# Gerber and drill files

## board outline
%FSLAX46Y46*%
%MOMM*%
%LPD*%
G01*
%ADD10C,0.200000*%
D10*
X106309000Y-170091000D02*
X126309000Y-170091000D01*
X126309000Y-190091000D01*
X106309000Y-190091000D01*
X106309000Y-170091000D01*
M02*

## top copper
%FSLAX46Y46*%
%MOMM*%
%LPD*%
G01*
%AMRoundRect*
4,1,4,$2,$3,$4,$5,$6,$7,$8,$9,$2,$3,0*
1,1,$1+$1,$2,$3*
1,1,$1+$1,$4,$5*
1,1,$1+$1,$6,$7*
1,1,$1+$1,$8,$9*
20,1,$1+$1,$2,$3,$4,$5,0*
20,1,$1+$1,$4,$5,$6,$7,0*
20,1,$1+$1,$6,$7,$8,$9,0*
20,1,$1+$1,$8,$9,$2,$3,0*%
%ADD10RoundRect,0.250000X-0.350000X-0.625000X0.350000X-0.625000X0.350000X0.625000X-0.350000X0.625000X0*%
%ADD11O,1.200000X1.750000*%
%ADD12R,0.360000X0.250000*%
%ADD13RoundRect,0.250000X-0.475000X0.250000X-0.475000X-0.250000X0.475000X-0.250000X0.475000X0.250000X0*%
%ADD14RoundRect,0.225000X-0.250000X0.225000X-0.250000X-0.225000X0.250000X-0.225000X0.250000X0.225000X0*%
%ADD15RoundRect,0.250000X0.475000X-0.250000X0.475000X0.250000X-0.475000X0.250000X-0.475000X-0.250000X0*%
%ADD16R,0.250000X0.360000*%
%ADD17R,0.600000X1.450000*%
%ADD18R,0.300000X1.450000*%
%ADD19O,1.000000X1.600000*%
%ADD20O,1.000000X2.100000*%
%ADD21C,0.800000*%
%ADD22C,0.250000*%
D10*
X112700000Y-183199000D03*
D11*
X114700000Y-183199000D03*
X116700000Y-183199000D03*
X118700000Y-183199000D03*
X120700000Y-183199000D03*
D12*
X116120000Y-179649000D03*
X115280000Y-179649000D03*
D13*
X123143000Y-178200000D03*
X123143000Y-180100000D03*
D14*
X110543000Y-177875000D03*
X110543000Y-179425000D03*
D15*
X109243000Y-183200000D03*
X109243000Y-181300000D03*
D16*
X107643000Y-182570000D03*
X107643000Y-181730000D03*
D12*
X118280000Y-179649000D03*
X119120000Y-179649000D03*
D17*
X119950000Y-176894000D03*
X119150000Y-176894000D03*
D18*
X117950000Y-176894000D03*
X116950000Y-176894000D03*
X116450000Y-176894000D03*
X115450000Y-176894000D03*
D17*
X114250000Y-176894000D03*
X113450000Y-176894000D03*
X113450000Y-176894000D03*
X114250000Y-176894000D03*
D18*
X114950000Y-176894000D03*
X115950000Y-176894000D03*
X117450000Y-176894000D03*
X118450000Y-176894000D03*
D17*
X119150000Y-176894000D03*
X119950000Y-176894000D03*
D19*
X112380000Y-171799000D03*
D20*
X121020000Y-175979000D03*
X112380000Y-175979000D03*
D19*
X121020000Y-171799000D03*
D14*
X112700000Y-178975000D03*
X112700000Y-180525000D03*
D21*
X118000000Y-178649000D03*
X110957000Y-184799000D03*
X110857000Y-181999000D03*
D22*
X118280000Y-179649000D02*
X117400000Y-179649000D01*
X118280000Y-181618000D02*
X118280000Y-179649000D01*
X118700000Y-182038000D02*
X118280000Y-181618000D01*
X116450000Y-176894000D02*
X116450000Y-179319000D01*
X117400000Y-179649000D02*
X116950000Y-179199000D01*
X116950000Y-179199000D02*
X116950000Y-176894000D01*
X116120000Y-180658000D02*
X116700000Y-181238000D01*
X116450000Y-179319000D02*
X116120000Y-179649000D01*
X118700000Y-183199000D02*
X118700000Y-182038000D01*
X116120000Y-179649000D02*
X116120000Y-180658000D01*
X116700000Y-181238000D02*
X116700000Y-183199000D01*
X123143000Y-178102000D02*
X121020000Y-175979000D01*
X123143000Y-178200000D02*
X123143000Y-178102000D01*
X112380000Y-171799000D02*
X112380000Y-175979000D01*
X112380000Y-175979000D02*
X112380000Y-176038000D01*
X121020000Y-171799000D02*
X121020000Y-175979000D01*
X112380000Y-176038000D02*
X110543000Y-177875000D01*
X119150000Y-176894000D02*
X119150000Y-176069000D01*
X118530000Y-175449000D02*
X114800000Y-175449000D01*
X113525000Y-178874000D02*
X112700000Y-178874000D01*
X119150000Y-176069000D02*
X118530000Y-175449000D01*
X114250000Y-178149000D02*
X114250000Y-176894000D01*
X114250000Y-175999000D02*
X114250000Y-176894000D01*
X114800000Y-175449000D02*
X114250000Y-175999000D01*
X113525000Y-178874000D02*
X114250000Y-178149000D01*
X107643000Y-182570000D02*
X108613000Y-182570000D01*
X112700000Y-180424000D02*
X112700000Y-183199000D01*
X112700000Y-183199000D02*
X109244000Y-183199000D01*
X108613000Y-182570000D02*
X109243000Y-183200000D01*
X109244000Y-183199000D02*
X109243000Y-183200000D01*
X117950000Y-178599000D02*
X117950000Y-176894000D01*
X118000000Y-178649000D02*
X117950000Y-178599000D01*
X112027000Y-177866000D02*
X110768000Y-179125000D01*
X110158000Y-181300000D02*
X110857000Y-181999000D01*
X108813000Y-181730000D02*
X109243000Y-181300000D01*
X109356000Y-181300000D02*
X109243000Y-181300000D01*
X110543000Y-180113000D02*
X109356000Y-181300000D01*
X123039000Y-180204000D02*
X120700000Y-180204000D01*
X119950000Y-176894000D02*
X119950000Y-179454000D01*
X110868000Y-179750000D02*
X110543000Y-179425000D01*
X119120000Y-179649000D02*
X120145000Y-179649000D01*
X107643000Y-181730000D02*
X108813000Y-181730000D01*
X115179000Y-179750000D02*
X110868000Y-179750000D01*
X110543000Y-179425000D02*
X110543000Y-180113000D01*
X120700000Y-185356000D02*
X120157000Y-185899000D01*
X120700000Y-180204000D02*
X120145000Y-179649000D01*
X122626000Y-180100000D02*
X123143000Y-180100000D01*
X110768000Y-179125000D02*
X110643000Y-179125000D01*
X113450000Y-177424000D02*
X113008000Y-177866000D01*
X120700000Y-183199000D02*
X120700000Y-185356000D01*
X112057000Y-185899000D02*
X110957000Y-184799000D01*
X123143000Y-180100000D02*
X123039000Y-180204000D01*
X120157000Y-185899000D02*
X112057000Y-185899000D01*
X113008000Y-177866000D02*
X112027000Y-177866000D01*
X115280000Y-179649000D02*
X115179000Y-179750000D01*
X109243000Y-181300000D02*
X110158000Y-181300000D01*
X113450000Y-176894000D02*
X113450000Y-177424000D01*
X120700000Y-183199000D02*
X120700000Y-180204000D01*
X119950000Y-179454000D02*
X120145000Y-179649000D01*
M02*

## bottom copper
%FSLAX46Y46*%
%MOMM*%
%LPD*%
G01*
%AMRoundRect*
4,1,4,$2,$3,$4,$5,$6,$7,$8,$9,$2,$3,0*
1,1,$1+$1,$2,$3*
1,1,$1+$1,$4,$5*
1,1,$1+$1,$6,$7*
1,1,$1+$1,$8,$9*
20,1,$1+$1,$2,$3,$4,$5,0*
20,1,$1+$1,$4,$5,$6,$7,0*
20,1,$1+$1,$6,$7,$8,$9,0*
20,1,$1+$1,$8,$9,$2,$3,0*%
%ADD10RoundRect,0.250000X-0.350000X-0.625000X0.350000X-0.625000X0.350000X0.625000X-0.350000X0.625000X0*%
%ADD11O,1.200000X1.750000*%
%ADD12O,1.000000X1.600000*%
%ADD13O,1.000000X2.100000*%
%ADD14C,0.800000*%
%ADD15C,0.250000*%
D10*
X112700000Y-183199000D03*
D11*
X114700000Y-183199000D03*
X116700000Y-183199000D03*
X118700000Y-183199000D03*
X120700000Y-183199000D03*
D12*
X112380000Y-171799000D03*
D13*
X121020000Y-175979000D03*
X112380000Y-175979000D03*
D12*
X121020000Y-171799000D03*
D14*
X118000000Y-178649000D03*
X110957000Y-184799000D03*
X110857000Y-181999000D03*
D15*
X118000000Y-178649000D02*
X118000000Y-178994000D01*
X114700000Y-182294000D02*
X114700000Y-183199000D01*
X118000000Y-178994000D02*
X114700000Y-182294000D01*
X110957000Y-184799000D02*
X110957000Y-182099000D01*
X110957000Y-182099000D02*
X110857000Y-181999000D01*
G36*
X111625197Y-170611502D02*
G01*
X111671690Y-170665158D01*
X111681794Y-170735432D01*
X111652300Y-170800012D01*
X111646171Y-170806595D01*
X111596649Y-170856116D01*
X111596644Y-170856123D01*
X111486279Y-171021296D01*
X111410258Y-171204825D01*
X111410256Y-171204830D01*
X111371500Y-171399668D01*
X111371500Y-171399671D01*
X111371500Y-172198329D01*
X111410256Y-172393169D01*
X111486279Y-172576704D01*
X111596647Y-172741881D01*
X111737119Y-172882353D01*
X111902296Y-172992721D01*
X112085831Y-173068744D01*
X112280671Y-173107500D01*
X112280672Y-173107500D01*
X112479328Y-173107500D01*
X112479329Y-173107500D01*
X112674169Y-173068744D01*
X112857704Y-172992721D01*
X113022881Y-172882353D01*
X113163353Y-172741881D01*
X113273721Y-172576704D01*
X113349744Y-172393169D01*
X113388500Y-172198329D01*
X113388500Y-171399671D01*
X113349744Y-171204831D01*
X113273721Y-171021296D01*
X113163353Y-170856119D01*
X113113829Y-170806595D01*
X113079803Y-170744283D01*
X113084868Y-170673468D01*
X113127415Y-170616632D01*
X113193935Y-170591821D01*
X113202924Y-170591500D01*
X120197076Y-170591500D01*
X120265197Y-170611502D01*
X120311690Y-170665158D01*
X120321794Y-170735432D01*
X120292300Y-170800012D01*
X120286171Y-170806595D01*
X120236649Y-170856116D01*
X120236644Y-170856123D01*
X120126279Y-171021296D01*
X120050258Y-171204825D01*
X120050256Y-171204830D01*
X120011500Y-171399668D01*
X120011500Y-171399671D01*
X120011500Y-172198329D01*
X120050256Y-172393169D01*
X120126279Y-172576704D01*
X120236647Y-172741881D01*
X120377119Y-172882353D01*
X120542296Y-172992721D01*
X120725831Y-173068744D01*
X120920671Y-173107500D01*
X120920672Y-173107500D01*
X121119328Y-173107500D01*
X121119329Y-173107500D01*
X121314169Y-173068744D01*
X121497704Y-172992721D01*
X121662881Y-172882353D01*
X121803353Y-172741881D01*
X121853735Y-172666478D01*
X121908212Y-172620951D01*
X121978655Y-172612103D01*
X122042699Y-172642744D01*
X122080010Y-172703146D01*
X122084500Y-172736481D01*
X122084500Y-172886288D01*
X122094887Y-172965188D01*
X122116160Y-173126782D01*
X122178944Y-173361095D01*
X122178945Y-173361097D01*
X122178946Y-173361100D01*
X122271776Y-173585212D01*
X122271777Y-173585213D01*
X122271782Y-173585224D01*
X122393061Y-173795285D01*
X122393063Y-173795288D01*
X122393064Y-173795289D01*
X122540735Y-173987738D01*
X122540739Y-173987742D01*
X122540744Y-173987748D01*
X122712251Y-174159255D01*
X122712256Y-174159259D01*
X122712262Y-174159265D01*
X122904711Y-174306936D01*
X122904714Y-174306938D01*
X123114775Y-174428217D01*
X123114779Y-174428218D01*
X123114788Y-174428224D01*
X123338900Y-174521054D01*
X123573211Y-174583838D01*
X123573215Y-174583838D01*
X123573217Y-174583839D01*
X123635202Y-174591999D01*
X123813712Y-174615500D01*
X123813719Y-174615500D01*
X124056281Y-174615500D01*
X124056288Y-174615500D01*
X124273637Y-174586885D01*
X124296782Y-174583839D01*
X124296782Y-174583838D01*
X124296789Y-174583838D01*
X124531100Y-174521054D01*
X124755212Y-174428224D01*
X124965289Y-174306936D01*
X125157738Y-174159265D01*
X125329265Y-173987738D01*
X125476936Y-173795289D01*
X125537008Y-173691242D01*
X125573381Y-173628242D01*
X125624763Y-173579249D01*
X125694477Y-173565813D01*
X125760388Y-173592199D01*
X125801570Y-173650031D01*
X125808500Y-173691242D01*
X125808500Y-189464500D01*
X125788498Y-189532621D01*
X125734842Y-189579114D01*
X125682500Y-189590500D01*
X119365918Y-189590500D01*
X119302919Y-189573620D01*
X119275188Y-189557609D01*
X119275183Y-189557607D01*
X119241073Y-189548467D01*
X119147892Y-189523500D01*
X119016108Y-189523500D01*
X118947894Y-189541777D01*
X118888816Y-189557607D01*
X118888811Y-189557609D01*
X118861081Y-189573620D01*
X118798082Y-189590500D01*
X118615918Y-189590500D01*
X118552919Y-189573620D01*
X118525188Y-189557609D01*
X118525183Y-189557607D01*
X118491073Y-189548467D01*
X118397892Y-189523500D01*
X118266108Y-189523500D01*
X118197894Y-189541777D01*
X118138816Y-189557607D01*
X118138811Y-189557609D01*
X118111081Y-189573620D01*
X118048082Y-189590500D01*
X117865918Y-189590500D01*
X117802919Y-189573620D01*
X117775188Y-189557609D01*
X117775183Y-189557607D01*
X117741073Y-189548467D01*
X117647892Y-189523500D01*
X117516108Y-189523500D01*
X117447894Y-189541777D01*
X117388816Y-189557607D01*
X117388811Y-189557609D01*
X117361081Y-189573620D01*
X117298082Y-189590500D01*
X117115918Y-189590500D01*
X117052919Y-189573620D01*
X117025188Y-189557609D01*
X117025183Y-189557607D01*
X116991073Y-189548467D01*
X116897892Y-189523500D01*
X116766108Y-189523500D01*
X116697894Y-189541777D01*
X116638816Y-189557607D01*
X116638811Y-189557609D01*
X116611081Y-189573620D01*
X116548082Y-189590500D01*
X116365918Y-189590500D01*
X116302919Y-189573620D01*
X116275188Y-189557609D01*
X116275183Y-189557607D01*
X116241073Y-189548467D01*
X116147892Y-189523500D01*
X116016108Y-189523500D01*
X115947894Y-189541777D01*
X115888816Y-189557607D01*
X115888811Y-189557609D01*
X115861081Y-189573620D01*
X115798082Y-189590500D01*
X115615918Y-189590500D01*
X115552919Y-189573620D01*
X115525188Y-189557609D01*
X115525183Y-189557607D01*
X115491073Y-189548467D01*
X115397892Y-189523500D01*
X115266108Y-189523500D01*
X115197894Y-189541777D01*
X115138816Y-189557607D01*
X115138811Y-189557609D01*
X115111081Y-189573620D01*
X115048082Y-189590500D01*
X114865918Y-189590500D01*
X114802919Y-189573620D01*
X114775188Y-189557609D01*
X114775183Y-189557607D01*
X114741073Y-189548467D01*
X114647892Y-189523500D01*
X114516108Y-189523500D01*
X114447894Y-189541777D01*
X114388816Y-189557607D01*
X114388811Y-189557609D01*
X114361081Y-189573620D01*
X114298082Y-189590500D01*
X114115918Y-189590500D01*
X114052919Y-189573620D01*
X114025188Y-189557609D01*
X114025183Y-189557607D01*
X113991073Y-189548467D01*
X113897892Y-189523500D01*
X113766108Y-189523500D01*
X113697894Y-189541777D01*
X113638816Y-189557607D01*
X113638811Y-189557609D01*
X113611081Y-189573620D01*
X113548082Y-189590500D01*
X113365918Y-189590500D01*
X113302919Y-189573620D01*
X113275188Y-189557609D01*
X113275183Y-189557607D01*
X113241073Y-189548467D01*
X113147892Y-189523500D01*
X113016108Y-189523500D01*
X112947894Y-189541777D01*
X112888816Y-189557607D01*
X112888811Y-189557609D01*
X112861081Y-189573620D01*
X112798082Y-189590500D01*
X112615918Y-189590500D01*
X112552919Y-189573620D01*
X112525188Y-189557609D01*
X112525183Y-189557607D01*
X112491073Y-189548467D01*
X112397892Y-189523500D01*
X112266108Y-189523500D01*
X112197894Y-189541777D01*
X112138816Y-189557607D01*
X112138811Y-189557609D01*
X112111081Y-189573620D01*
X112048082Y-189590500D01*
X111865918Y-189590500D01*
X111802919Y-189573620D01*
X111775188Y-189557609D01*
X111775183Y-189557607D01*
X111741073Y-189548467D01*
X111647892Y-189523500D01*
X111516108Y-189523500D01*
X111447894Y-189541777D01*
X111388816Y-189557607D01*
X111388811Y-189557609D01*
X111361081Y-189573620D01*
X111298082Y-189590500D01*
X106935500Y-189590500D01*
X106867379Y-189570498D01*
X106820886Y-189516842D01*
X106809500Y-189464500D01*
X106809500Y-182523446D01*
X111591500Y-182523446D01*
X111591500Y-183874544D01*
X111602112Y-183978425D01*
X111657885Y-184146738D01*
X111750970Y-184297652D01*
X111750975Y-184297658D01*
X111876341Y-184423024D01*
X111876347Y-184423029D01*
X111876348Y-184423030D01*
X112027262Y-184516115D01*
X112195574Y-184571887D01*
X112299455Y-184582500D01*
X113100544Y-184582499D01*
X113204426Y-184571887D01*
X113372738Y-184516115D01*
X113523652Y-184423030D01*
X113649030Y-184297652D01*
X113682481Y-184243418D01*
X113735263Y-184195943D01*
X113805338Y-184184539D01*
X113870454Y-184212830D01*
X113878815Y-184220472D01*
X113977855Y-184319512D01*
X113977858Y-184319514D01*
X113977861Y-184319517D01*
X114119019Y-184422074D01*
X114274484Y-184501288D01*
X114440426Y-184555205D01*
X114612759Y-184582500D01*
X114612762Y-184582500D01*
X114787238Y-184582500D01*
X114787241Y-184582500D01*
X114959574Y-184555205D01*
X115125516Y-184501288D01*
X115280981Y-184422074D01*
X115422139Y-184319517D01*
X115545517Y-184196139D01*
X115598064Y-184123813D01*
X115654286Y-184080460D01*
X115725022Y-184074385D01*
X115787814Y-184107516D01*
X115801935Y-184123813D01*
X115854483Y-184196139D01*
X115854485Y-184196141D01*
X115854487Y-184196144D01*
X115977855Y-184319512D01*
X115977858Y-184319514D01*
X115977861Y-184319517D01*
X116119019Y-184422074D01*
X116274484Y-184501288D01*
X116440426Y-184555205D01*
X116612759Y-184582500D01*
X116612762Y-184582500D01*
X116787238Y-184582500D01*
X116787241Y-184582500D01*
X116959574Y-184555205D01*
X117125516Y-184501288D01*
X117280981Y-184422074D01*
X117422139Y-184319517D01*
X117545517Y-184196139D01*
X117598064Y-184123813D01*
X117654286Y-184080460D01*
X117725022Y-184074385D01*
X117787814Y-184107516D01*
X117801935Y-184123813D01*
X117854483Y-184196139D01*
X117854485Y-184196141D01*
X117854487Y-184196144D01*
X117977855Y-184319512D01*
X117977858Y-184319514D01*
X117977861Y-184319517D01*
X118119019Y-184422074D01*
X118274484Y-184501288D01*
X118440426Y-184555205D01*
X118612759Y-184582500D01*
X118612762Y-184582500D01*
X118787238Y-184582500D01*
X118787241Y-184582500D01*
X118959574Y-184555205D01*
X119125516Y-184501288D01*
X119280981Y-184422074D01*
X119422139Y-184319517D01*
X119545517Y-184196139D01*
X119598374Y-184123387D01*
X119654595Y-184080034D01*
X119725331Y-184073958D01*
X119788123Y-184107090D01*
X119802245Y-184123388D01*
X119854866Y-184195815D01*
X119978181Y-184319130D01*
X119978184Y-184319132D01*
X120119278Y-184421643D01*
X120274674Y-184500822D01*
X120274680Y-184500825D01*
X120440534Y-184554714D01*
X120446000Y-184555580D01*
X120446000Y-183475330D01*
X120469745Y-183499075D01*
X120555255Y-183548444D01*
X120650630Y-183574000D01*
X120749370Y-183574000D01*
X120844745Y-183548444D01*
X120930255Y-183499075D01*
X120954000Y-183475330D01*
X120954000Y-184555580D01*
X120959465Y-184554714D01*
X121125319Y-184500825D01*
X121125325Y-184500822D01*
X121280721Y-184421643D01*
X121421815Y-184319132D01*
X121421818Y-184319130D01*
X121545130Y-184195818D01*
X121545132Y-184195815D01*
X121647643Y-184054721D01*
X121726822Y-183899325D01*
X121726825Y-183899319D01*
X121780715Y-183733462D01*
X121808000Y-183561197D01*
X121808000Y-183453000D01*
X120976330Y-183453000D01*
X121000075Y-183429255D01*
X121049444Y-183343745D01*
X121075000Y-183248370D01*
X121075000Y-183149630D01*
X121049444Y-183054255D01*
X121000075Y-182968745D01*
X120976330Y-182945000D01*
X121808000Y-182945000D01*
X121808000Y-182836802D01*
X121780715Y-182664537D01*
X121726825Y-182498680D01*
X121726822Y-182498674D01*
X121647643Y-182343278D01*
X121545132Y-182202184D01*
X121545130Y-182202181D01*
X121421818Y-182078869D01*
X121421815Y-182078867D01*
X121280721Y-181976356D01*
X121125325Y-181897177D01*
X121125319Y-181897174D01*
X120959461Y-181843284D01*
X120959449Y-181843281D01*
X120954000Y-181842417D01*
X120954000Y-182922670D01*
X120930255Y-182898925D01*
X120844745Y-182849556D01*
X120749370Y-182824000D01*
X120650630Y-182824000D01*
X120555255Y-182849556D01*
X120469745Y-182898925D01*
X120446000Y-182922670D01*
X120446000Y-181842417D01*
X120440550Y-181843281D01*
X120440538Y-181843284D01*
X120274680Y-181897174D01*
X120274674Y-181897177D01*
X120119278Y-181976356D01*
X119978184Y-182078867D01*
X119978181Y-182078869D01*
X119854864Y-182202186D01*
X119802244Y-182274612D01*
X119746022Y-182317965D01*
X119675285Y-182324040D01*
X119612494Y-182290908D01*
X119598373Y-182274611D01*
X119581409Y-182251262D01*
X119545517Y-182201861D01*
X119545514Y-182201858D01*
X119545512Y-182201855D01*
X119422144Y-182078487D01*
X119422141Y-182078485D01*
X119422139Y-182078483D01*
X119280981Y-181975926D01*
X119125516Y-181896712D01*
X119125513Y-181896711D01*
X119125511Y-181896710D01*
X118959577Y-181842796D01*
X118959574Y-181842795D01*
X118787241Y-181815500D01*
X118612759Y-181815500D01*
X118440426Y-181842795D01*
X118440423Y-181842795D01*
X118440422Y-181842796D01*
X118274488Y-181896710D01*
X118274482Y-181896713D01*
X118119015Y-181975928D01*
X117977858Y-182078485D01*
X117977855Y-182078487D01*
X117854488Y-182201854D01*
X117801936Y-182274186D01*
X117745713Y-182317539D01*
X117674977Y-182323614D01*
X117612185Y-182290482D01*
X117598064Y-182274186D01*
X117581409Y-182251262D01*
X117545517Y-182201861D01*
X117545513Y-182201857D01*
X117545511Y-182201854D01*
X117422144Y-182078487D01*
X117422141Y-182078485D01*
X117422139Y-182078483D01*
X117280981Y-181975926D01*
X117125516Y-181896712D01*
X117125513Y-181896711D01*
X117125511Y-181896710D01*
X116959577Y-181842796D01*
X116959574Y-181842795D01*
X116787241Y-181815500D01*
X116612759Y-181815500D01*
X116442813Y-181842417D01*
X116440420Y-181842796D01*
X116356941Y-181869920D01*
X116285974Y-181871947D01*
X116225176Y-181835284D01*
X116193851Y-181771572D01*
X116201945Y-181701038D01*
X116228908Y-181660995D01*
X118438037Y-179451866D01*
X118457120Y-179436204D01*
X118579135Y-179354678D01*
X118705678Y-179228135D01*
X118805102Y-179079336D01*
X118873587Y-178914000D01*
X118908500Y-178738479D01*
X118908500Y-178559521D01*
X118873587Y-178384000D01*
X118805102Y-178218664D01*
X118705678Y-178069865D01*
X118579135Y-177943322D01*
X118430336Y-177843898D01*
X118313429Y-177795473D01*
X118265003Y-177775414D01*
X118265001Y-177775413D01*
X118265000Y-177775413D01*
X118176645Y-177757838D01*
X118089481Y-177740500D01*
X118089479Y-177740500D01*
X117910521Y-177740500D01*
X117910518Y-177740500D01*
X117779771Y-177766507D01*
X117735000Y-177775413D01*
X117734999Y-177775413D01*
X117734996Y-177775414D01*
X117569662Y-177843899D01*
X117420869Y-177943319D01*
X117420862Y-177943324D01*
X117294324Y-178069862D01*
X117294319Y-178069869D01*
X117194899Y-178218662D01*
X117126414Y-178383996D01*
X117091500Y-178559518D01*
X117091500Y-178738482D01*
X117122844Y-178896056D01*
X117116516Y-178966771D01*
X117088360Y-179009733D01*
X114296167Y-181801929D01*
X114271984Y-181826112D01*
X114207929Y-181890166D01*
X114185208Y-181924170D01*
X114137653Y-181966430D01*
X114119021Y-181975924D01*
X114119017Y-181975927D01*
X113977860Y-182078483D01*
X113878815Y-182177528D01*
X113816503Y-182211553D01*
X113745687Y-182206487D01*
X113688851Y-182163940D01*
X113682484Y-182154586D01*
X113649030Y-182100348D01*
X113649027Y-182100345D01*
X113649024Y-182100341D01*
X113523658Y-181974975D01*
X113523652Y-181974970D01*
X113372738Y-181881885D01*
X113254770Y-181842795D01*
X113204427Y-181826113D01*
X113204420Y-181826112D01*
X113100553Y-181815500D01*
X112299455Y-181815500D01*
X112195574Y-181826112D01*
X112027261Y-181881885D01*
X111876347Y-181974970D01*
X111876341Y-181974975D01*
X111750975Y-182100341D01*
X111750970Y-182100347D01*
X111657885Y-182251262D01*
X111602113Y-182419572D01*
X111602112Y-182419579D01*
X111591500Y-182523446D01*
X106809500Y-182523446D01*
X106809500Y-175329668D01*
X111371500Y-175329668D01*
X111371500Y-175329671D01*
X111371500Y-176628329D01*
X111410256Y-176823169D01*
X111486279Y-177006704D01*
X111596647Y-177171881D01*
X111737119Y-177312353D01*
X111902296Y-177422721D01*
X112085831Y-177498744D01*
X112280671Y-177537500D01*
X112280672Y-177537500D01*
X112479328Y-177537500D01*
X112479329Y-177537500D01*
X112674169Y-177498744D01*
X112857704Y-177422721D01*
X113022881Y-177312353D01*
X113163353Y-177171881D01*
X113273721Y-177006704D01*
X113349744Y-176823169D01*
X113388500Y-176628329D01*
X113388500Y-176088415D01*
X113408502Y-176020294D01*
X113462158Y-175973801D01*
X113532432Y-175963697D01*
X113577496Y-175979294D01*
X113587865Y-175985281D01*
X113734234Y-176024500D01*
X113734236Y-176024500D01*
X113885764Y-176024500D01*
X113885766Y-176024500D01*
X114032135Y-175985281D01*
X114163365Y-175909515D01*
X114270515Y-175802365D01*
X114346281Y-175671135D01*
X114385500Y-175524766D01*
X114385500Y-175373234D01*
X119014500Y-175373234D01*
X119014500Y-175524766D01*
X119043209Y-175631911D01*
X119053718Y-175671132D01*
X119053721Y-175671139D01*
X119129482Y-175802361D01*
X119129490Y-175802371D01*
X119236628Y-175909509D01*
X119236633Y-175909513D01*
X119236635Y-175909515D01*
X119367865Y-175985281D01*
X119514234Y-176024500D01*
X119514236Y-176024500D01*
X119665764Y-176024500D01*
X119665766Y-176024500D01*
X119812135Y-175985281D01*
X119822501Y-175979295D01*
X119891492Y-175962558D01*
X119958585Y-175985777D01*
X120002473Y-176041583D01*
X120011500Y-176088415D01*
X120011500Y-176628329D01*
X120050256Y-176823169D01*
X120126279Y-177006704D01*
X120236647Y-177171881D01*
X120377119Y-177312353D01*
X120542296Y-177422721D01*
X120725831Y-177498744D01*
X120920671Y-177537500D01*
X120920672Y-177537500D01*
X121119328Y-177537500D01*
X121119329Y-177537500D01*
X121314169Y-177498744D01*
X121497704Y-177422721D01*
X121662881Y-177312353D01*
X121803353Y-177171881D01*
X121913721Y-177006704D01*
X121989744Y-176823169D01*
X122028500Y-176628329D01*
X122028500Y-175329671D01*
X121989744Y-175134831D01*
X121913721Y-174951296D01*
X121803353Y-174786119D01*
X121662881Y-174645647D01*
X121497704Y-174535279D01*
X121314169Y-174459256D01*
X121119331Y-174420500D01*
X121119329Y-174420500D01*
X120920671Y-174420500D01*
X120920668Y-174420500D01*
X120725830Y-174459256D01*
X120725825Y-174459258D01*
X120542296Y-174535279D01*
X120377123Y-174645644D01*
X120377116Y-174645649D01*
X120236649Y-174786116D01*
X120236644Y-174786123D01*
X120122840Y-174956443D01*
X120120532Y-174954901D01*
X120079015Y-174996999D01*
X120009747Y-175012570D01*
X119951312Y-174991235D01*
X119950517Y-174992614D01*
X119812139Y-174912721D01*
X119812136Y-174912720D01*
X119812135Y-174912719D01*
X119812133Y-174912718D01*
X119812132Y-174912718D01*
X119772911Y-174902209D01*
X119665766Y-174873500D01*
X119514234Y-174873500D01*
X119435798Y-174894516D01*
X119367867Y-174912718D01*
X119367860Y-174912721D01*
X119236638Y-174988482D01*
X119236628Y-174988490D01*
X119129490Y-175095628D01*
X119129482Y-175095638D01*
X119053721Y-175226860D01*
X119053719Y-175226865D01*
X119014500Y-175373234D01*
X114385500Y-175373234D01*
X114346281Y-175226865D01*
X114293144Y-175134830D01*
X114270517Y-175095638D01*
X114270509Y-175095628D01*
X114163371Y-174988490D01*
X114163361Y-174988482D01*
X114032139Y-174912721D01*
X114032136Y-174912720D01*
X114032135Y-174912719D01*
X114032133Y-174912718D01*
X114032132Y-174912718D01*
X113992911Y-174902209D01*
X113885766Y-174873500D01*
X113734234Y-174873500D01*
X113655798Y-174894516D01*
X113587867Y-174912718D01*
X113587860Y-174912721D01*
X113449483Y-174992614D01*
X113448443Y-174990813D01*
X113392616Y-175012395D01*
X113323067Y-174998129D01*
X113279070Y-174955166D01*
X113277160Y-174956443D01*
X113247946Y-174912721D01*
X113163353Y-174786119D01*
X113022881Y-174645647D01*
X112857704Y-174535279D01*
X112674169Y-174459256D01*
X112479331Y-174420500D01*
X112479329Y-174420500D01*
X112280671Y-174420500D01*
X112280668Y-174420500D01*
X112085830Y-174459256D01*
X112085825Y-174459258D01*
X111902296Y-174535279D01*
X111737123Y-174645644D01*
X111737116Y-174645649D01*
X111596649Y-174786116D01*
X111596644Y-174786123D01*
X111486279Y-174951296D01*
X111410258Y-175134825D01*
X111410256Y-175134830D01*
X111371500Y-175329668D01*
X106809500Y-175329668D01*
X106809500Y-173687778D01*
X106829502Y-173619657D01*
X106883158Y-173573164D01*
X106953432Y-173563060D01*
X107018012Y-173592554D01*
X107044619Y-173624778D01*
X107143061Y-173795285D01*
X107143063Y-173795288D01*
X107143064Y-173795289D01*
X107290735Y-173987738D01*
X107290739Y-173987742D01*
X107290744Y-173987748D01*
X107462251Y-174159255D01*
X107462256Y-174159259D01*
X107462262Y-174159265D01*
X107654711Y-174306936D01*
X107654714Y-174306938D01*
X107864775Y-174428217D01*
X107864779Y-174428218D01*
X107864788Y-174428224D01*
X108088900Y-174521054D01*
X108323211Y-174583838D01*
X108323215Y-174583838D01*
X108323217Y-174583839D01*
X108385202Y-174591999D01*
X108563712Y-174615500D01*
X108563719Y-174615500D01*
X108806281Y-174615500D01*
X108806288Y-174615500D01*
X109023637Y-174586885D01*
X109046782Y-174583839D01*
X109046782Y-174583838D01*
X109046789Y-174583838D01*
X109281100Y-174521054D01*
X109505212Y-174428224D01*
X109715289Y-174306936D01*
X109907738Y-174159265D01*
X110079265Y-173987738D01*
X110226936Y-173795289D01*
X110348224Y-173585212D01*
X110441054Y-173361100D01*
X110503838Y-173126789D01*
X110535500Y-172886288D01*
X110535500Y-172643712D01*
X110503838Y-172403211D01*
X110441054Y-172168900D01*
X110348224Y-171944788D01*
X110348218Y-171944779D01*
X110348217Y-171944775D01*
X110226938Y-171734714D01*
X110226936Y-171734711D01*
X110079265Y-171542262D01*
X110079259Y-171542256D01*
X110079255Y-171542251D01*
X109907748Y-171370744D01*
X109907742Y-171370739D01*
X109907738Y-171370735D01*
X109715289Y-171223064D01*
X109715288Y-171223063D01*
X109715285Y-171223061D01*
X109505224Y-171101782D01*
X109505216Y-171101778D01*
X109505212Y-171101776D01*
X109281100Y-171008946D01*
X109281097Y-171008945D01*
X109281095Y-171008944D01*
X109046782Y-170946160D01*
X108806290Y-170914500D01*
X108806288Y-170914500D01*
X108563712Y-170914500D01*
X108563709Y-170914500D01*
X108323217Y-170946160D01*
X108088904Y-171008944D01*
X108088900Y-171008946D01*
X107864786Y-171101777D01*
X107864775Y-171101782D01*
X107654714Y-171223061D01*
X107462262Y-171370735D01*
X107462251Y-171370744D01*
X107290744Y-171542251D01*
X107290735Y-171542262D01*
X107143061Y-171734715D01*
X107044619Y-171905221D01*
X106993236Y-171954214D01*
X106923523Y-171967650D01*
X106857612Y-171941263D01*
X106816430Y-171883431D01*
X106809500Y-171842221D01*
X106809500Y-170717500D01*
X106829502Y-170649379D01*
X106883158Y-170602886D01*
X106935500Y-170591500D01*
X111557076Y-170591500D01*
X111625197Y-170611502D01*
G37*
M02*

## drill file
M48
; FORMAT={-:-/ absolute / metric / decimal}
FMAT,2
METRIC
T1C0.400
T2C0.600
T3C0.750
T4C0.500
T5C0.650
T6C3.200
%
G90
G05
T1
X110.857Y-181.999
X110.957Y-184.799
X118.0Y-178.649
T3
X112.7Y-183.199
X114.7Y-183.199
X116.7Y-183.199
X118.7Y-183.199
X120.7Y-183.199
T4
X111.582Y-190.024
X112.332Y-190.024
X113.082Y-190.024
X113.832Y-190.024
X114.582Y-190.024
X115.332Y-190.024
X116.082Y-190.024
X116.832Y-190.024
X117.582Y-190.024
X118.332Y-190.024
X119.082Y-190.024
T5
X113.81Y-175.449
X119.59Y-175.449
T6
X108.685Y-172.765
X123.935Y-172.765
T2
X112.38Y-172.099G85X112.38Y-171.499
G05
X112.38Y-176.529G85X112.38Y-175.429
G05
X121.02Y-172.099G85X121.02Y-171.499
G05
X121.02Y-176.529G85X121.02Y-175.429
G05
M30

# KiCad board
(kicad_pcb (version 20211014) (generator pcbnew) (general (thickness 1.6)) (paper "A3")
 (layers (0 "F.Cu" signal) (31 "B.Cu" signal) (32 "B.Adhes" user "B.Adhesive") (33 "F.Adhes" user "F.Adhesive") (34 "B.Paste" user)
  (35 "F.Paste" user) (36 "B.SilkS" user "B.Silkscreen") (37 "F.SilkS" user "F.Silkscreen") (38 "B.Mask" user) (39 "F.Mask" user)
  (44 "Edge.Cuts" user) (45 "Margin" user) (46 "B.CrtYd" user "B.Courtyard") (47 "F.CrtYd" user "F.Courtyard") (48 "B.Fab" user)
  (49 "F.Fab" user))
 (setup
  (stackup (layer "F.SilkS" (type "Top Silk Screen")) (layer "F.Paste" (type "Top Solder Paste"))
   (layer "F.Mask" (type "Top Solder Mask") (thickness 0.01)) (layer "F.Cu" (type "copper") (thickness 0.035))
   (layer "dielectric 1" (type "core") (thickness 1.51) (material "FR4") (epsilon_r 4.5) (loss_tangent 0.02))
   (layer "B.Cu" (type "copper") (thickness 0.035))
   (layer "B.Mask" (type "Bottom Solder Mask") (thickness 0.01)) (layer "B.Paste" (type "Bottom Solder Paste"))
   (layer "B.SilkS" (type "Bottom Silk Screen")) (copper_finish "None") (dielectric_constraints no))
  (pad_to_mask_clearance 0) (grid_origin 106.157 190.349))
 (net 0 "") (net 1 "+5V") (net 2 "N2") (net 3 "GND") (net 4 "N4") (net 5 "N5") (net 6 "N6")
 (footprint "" (layer "F.Cu") (at 111.582 190.024 90)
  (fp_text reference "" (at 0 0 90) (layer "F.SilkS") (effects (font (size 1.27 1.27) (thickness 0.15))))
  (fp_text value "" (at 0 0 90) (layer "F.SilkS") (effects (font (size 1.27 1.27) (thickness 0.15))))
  (pad "" np_thru_hole circle locked (at 0 0 180) (size 0.5 0.5) (drill 0.5) (layers F&B.Cu *.Mask)))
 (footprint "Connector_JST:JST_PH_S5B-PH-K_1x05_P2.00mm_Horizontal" (layer "F.Cu") (at 112.7 183.199)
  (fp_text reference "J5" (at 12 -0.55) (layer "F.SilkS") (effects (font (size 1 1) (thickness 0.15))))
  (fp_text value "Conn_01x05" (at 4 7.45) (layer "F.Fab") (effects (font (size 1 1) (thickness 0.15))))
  (pad "1" thru_hole roundrect (at 0 0) (size 1.2 1.75) (drill 0.75) (layers F&B.Cu *.Mask) (roundrect_rratio 0.2083333333) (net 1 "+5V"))
  (pad "2" thru_hole oval (at 2 0) (size 1.2 1.75) (drill 0.75) (layers F&B.Cu *.Mask) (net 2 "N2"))
  (pad "3" thru_hole oval (at 4 0) (size 1.2 1.75) (drill 0.75) (layers F&B.Cu *.Mask))
  (pad "4" thru_hole oval (at 6 0) (size 1.2 1.75) (drill 0.75) (layers F&B.Cu *.Mask))
  (pad "5" thru_hole oval (at 8 0) (size 1.2 1.75) (drill 0.75) (layers F&B.Cu *.Mask) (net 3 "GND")))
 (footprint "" (layer "F.Cu") (at 118.332 190.024 90)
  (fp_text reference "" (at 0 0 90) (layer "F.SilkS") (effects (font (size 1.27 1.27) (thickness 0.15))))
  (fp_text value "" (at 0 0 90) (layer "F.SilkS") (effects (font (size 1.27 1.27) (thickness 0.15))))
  (pad "" np_thru_hole circle locked (at 0 0 180) (size 0.5 0.5) (drill 0.5) (layers F&B.Cu *.Mask)))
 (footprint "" (layer "F.Cu") (at 113.082 190.024 90)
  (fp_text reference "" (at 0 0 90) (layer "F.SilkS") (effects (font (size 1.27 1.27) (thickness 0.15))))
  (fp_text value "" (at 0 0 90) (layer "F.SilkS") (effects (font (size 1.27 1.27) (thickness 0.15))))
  (pad "" np_thru_hole circle locked (at 0 0 180) (size 0.5 0.5) (drill 0.5) (layers F&B.Cu *.Mask)))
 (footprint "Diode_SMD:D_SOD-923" (layer "F.Cu") (at 115.7 179.649 180)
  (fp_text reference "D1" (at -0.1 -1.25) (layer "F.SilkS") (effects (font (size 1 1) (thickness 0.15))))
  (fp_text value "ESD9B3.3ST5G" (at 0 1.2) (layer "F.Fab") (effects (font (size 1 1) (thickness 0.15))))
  (pad "1" smd rect (at -0.42 0) (size 0.36 0.25) (layers "F.Cu" "F.Paste" "F.Mask"))
  (pad "2" smd rect (at 0.42 0) (size 0.36 0.25) (layers "F.Cu" "F.Paste" "F.Mask") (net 3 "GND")))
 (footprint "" (layer "F.Cu") (at 112.332 190.024 90)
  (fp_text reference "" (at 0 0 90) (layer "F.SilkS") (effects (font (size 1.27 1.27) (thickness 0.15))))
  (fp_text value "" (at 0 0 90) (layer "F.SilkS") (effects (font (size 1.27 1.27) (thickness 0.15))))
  (pad "" np_thru_hole circle locked (at 0 0 180) (size 0.5 0.5) (drill 0.5) (layers F&B.Cu *.Mask)))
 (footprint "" (layer "F.Cu") (at 116.832 190.024 90)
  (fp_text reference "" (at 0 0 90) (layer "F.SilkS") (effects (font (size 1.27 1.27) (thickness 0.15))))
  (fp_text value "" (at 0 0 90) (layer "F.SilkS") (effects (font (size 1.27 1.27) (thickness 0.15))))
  (pad "" np_thru_hole circle locked (at 0 0 180) (size 0.5 0.5) (drill 0.5) (layers F&B.Cu *.Mask)))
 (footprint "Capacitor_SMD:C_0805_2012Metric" (layer "F.Cu") (at 123.143 179.15 -90)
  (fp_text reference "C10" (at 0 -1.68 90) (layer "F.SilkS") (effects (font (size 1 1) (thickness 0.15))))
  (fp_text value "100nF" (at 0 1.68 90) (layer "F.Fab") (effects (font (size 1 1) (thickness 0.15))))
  (pad "1" smd roundrect (at -0.95 0 270) (size 1 1.45) (layers "F.Cu" "F.Paste" "F.Mask") (roundrect_rratio 0.25) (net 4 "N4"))
  (pad "2" smd roundrect (at 0.95 0 270) (size 1 1.45) (layers "F.Cu" "F.Paste" "F.Mask") (roundrect_rratio 0.25) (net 3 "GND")))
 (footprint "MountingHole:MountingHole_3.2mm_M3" (layer "F.Cu") (at 124.065 172.615 180)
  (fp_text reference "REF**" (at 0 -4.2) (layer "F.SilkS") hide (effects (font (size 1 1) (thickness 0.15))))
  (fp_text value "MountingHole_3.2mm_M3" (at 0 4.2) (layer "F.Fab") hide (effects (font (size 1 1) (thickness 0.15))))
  (pad "" np_thru_hole circle (at 0.13 -0.15 180) (size 3.2 3.2) (drill 3.2) (layers F&B.Cu *.Mask)))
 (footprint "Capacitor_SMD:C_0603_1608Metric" (layer "F.Cu") (at 110.543 178.65 -90)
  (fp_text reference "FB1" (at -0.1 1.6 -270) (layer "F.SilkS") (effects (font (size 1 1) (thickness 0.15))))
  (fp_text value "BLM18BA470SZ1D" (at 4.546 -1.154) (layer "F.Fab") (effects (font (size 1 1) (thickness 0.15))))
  (pad "1" smd roundrect (at -0.775 0 270) (size 0.9 0.95) (layers "F.Cu" "F.Paste" "F.Mask") (roundrect_rratio 0.25) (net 4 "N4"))
  (pad "2" smd roundrect (at 0.775 0 270) (size 0.9 0.95) (layers "F.Cu" "F.Paste" "F.Mask") (roundrect_rratio 0.25) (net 3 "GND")))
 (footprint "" (layer "F.Cu") (at 115.332 190.024 90)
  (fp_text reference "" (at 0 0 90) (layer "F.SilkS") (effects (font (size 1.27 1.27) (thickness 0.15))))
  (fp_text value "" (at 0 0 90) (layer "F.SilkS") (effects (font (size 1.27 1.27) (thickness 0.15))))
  (pad "" np_thru_hole circle locked (at 0 0 180) (size 0.5 0.5) (drill 0.5) (layers F&B.Cu *.Mask)))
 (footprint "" (layer "F.Cu") (at 119.082 190.024 90)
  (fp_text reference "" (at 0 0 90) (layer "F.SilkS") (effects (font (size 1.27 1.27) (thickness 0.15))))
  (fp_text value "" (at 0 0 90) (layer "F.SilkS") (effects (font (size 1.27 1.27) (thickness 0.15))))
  (pad "" np_thru_hole circle locked (at 0 0 180) (size 0.5 0.5) (drill 0.5) (layers F&B.Cu *.Mask)))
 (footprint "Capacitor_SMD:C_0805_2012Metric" (layer "F.Cu") (at 109.243 182.25 90)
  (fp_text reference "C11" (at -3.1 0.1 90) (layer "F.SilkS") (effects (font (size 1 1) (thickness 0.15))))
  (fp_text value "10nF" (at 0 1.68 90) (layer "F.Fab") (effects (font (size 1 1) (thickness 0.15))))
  (pad "1" smd roundrect (at -0.95 0 90) (size 1 1.45) (layers "F.Cu" "F.Paste" "F.Mask") (roundrect_rratio 0.25) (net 1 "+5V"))
  (pad "2" smd roundrect (at 0.95 0 90) (size 1 1.45) (layers "F.Cu" "F.Paste" "F.Mask") (roundrect_rratio 0.25) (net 3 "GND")))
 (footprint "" (layer "F.Cu") (at 116.082 190.024 90)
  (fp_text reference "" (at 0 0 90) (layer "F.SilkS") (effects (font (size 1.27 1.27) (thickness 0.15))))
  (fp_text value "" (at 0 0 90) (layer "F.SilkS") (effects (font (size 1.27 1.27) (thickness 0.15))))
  (pad "" np_thru_hole circle locked (at 0 0 180) (size 0.5 0.5) (drill 0.5) (layers F&B.Cu *.Mask)))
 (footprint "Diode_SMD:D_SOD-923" (layer "F.Cu") (at 107.643 182.15 90)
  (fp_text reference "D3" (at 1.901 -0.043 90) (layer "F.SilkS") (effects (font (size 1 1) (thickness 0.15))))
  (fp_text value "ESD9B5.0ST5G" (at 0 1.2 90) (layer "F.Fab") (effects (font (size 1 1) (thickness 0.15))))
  (pad "1" smd rect (at -0.42 0 270) (size 0.36 0.25) (layers "F.Cu" "F.Paste" "F.Mask") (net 1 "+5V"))
  (pad "2" smd rect (at 0.42 0 270) (size 0.36 0.25) (layers "F.Cu" "F.Paste" "F.Mask") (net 3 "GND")))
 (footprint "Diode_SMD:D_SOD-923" (layer "F.Cu") (at 118.7 179.649)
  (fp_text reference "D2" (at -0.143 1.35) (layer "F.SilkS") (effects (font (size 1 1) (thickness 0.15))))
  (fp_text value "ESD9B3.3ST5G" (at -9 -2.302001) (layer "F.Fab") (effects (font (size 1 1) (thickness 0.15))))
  (pad "1" smd rect (at -0.42 0 180) (size 0.36 0.25) (layers "F.Cu" "F.Paste" "F.Mask"))
  (pad "2" smd rect (at 0.42 0 180) (size 0.36 0.25) (layers "F.Cu" "F.Paste" "F.Mask") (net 3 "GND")))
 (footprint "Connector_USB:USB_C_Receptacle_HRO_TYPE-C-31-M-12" (layer "F.Cu") (at 116.7 172.849 180)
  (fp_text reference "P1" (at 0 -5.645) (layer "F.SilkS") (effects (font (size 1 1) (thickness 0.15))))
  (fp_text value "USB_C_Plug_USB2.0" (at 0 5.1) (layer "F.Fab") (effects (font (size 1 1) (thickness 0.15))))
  (pad "" np_thru_hole circle (at -2.89 -2.6 180) (size 0.65 0.65) (drill 0.65) (layers F&B.Cu *.Mask))
  (pad "" np_thru_hole circle (at 2.89 -2.6 180) (size 0.65 0.65) (drill 0.65) (layers F&B.Cu *.Mask))
  (pad "A1" smd rect (at -3.25 -4.045 180) (size 0.6 1.45) (layers "F.Cu" "F.Paste" "F.Mask") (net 3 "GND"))
  (pad "A4" smd rect (at -2.45 -4.045 180) (size 0.6 1.45) (layers "F.Cu" "F.Paste" "F.Mask") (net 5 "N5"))
  (pad "A5" smd rect (at -1.25 -4.045 180) (size 0.3 1.45) (layers "F.Cu" "F.Paste" "F.Mask") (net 2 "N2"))
  (pad "A6" smd rect (at -0.25 -4.045 180) (size 0.3 1.45) (layers "F.Cu" "F.Paste" "F.Mask"))
  (pad "A7" smd rect (at 0.25 -4.045 180) (size 0.3 1.45) (layers "F.Cu" "F.Paste" "F.Mask"))
  (pad "A8" smd rect (at 1.25 -4.045 180) (size 0.3 1.45) (layers "F.Cu" "F.Paste" "F.Mask"))
  (pad "A9" smd rect (at 2.45 -4.045 180) (size 0.6 1.45) (layers "F.Cu" "F.Paste" "F.Mask") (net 5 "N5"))
  (pad "A12" smd rect (at 3.25 -4.045 180) (size 0.6 1.45) (layers "F.Cu" "F.Paste" "F.Mask") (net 3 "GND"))
  (pad "B1" smd rect (at 3.25 -4.045 180) (size 0.6 1.45) (layers "F.Cu" "F.Paste" "F.Mask") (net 3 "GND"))
  (pad "B4" smd rect (at 2.45 -4.045 180) (size 0.6 1.45) (layers "F.Cu" "F.Paste" "F.Mask") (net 5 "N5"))
  (pad "B5" smd rect (at 1.75 -4.045 180) (size 0.3 1.45) (layers "F.Cu" "F.Paste" "F.Mask") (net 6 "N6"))
  (pad "B6" smd rect (at 0.75 -4.045 180) (size 0.3 1.45) (layers "F.Cu" "F.Paste" "F.Mask"))
  (pad "B7" smd rect (at -0.75 -4.045 180) (size 0.3 1.45) (layers "F.Cu" "F.Paste" "F.Mask"))
  (pad "B8" smd rect (at -1.75 -4.045 180) (size 0.3 1.45) (layers "F.Cu" "F.Paste" "F.Mask"))
  (pad "B9" smd rect (at -2.45 -4.045 180) (size 0.6 1.45) (layers "F.Cu" "F.Paste" "F.Mask") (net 5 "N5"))
  (pad "B12" smd rect (at -3.25 -4.045 180) (size 0.6 1.45) (layers "F.Cu" "F.Paste" "F.Mask") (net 3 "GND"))
  (pad "S1" thru_hole oval (at 4.32 1.05 180) (size 1 1.6) (drill oval 0.6 1.2) (layers F&B.Cu *.Mask) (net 4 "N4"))
  (pad "S1" thru_hole oval (at -4.32 -3.13 180) (size 1 2.1) (drill oval 0.6 1.7) (layers F&B.Cu *.Mask) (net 4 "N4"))
  (pad "S1" thru_hole oval (at 4.32 -3.13 180) (size 1 2.1) (drill oval 0.6 1.7) (layers F&B.Cu *.Mask) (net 4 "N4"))
  (pad "S1" thru_hole oval (at -4.32 1.05 180) (size 1 1.6) (drill oval 0.6 1.2) (layers F&B.Cu *.Mask) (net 4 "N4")))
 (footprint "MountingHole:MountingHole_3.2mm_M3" (layer "F.Cu") (at 108.885 172.715 180)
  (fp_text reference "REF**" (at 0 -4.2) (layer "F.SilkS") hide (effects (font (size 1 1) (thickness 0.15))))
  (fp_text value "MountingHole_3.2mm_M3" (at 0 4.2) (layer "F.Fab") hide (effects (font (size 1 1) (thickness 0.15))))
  (pad "" np_thru_hole circle (at 0.2 -0.05 180) (size 3.2 3.2) (drill 3.2) (layers F&B.Cu *.Mask)))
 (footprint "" (layer "F.Cu") (at 114.582 190.024 90)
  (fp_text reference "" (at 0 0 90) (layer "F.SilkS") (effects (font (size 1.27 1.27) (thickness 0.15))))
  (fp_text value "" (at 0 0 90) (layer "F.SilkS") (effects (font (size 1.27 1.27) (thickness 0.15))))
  (pad "" np_thru_hole circle locked (at 0 0 180) (size 0.5 0.5) (drill 0.5) (layers F&B.Cu *.Mask)))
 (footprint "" (layer "F.Cu") (at 117.582 190.024 90)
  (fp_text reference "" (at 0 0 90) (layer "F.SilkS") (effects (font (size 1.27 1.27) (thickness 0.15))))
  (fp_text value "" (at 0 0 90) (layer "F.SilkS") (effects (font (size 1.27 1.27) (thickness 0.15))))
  (pad "" np_thru_hole circle locked (at 0 0 180) (size 0.5 0.5) (drill 0.5) (layers F&B.Cu *.Mask)))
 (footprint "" (layer "F.Cu") (at 113.832 190.024 90)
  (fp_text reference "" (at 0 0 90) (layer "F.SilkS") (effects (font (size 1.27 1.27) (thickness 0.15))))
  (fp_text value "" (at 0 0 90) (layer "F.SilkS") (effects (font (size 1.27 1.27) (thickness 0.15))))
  (pad "" np_thru_hole circle locked (at 0 0 180) (size 0.5 0.5) (drill 0.5) (layers F&B.Cu *.Mask)))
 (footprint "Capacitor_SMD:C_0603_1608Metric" (layer "F.Cu") (at 112.7 179.75 -90)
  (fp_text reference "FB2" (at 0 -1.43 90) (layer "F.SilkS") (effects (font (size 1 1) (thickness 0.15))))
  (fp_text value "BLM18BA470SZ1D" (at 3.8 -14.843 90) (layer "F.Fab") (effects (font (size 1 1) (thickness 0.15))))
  (pad "1" smd roundrect (at -0.775 0 270) (size 0.9 0.95) (layers "F.Cu" "F.Paste" "F.Mask") (roundrect_rratio 0.25) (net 5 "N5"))
  (pad "2" smd roundrect (at 0.775 0 270) (size 0.9 0.95) (layers "F.Cu" "F.Paste" "F.Mask") (roundrect_rratio 0.25) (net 1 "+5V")))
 (gr_rect (start 106.309 170.091) (end 126.309 190.091) (layer "Edge.Cuts") (width 0.2) (fill none))
 (segment (start 118.28 179.649) (end 117.4 179.649) (width 0.25) (layer "F.Cu") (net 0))
 (segment (start 118.28 181.618) (end 118.28 179.649) (width 0.25) (layer "F.Cu") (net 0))
 (segment (start 118.7 182.038) (end 118.28 181.618) (width 0.25) (layer "F.Cu") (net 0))
 (segment (start 116.45 176.894) (end 116.45 179.319) (width 0.25) (layer "F.Cu") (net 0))
 (segment (start 117.4 179.649) (end 116.95 179.199) (width 0.25) (layer "F.Cu") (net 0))
 (segment (start 116.95 179.199) (end 116.95 176.894) (width 0.25) (layer "F.Cu") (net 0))
 (segment (start 116.12 180.658) (end 116.7 181.238) (width 0.25) (layer "F.Cu") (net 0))
 (segment (start 116.45 179.319) (end 116.12 179.649) (width 0.25) (layer "F.Cu") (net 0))
 (segment (start 118.7 183.199) (end 118.7 182.038) (width 0.25) (layer "F.Cu") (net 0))
 (segment (start 116.12 179.649) (end 116.12 180.658) (width 0.25) (layer "F.Cu") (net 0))
 (segment (start 116.7 181.238) (end 116.7 183.199) (width 0.25) (layer "F.Cu") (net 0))
 (segment (start 123.143 178.102) (end 121.02 175.979) (width 0.25) (layer "F.Cu") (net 4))
 (segment (start 123.143 178.2) (end 123.143 178.102) (width 0.25) (layer "F.Cu") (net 4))
 (segment (start 112.38 171.799) (end 112.38 175.979) (width 0.25) (layer "F.Cu") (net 4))
 (segment (start 112.38 175.979) (end 112.38 176.038) (width 0.25) (layer "F.Cu") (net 4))
 (segment (start 121.02 171.799) (end 121.02 175.979) (width 0.25) (layer "F.Cu") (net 4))
 (segment (start 112.38 176.038) (end 110.543 177.875) (width 0.25) (layer "F.Cu") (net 4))
 (segment (start 119.15 176.894) (end 119.15 176.069) (width 0.25) (layer "F.Cu") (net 5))
 (segment (start 118.53 175.449) (end 114.8 175.449) (width 0.25) (layer "F.Cu") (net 5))
 (segment (start 113.525 178.874) (end 112.7 178.874) (width 0.25) (layer "F.Cu") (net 5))
 (segment (start 119.15 176.069) (end 118.53 175.449) (width 0.25) (layer "F.Cu") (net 5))
 (segment (start 114.25 178.149) (end 114.25 176.894) (width 0.25) (layer "F.Cu") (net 5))
 (segment (start 114.25 175.999) (end 114.25 176.894) (width 0.25) (layer "F.Cu") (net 5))
 (segment (start 114.8 175.449) (end 114.25 175.999) (width 0.25) (layer "F.Cu") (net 5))
 (segment (start 113.525 178.874) (end 114.25 178.149) (width 0.25) (layer "F.Cu") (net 5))
 (segment (start 107.643 182.57) (end 108.613 182.57) (width 0.25) (layer "F.Cu") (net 1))
 (segment (start 112.7 180.424) (end 112.7 183.199) (width 0.25) (layer "F.Cu") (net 1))
 (segment (start 112.7 183.199) (end 109.244 183.199) (width 0.25) (layer "F.Cu") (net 1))
 (segment (start 108.613 182.57) (end 109.243 183.2) (width 0.25) (layer "F.Cu") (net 1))
 (segment (start 109.244 183.199) (end 109.243 183.2) (width 0.25) (layer "F.Cu") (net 1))
 (segment (start 117.95 178.599) (end 117.95 176.894) (width 0.25) (layer "F.Cu") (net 2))
 (segment (start 118 178.649) (end 117.95 178.599) (width 0.25) (layer "F.Cu") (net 2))
 (via (at 118 178.649) (size 0.8) (drill 0.4) (layers "F.Cu" "B.Cu") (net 2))
 (segment (start 118 178.649) (end 118 178.994) (width 0.25) (layer "B.Cu") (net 2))
 (segment (start 114.7 182.294) (end 114.7 183.199) (width 0.25) (layer "B.Cu") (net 2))
 (segment (start 118 178.994) (end 114.7 182.294) (width 0.25) (layer "B.Cu") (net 2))
 (segment (start 112.027 177.866) (end 110.768 179.125) (width 0.25) (layer "F.Cu") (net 3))
 (segment (start 110.158 181.3) (end 110.857 181.999) (width 0.25) (layer "F.Cu") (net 3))
 (segment (start 108.813 181.73) (end 109.243 181.3) (width 0.25) (layer "F.Cu") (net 3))
 (segment (start 109.356 181.3) (end 109.243 181.3) (width 0.25) (layer "F.Cu") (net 3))
 (segment (start 110.543 180.113) (end 109.356 181.3) (width 0.25) (layer "F.Cu") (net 3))
 (segment (start 123.039 180.204) (end 120.7 180.204) (width 0.25) (layer "F.Cu") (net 3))
 (segment (start 119.95 176.894) (end 119.95 179.454) (width 0.25) (layer "F.Cu") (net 3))
 (segment (start 110.868 179.75) (end 110.543 179.425) (width 0.25) (layer "F.Cu") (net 3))
 (segment (start 119.12 179.649) (end 120.145 179.649) (width 0.25) (layer "F.Cu") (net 3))
 (segment (start 107.643 181.73) (end 108.813 181.73) (width 0.25) (layer "F.Cu") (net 3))
 (segment (start 115.179 179.75) (end 110.868 179.75) (width 0.25) (layer "F.Cu") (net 3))
 (segment (start 110.543 179.425) (end 110.543 180.113) (width 0.25) (layer "F.Cu") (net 3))
 (segment (start 120.7 185.356) (end 120.157 185.899) (width 0.25) (layer "F.Cu") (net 3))
 (segment (start 120.7 180.204) (end 120.145 179.649) (width 0.25) (layer "F.Cu") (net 3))
 (segment (start 122.626 180.1) (end 123.143 180.1) (width 0.25) (layer "F.Cu") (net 3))
 (segment (start 110.768 179.125) (end 110.643 179.125) (width 0.25) (layer "F.Cu") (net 3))
 (segment (start 113.45 177.424) (end 113.008 177.866) (width 0.25) (layer "F.Cu") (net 3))
 (segment (start 120.7 183.199) (end 120.7 185.356) (width 0.25) (layer "F.Cu") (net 3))
 (segment (start 112.057 185.899) (end 110.957 184.799) (width 0.25) (layer "F.Cu") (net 3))
 (segment (start 123.143 180.1) (end 123.039 180.204) (width 0.25) (layer "F.Cu") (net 3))
 (segment (start 120.157 185.899) (end 112.057 185.899) (width 0.25) (layer "F.Cu") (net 3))
 (segment (start 113.008 177.866) (end 112.027 177.866) (width 0.25) (layer "F.Cu") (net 3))
 (segment (start 115.28 179.649) (end 115.179 179.75) (width 0.25) (layer "F.Cu") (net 3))
 (segment (start 109.243 181.3) (end 110.158 181.3) (width 0.25) (layer "F.Cu") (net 3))
 (segment (start 113.45 176.894) (end 113.45 177.424) (width 0.25) (layer "F.Cu") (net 3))
 (segment (start 120.7 183.199) (end 120.7 180.204) (width 0.25) (layer "F.Cu") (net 3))
 (segment (start 119.95 179.454) (end 120.145 179.649) (width 0.25) (layer "F.Cu") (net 3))
 (via (at 110.957 184.799) (size 0.8) (drill 0.4) (layers "F.Cu" "B.Cu") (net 3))
 (via (at 110.857 181.999) (size 0.8) (drill 0.4) (layers "F.Cu" "B.Cu") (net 3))
 (segment (start 110.957 184.799) (end 110.957 182.099) (width 0.25) (layer "B.Cu") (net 3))
 (segment (start 110.957 182.099) (end 110.857 181.999) (width 0.25) (layer "B.Cu") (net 3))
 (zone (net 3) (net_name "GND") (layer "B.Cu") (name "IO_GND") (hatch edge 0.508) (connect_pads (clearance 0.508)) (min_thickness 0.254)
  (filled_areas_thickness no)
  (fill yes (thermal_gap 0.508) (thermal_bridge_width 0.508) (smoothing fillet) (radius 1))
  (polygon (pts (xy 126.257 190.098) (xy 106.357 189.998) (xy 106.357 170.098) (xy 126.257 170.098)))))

